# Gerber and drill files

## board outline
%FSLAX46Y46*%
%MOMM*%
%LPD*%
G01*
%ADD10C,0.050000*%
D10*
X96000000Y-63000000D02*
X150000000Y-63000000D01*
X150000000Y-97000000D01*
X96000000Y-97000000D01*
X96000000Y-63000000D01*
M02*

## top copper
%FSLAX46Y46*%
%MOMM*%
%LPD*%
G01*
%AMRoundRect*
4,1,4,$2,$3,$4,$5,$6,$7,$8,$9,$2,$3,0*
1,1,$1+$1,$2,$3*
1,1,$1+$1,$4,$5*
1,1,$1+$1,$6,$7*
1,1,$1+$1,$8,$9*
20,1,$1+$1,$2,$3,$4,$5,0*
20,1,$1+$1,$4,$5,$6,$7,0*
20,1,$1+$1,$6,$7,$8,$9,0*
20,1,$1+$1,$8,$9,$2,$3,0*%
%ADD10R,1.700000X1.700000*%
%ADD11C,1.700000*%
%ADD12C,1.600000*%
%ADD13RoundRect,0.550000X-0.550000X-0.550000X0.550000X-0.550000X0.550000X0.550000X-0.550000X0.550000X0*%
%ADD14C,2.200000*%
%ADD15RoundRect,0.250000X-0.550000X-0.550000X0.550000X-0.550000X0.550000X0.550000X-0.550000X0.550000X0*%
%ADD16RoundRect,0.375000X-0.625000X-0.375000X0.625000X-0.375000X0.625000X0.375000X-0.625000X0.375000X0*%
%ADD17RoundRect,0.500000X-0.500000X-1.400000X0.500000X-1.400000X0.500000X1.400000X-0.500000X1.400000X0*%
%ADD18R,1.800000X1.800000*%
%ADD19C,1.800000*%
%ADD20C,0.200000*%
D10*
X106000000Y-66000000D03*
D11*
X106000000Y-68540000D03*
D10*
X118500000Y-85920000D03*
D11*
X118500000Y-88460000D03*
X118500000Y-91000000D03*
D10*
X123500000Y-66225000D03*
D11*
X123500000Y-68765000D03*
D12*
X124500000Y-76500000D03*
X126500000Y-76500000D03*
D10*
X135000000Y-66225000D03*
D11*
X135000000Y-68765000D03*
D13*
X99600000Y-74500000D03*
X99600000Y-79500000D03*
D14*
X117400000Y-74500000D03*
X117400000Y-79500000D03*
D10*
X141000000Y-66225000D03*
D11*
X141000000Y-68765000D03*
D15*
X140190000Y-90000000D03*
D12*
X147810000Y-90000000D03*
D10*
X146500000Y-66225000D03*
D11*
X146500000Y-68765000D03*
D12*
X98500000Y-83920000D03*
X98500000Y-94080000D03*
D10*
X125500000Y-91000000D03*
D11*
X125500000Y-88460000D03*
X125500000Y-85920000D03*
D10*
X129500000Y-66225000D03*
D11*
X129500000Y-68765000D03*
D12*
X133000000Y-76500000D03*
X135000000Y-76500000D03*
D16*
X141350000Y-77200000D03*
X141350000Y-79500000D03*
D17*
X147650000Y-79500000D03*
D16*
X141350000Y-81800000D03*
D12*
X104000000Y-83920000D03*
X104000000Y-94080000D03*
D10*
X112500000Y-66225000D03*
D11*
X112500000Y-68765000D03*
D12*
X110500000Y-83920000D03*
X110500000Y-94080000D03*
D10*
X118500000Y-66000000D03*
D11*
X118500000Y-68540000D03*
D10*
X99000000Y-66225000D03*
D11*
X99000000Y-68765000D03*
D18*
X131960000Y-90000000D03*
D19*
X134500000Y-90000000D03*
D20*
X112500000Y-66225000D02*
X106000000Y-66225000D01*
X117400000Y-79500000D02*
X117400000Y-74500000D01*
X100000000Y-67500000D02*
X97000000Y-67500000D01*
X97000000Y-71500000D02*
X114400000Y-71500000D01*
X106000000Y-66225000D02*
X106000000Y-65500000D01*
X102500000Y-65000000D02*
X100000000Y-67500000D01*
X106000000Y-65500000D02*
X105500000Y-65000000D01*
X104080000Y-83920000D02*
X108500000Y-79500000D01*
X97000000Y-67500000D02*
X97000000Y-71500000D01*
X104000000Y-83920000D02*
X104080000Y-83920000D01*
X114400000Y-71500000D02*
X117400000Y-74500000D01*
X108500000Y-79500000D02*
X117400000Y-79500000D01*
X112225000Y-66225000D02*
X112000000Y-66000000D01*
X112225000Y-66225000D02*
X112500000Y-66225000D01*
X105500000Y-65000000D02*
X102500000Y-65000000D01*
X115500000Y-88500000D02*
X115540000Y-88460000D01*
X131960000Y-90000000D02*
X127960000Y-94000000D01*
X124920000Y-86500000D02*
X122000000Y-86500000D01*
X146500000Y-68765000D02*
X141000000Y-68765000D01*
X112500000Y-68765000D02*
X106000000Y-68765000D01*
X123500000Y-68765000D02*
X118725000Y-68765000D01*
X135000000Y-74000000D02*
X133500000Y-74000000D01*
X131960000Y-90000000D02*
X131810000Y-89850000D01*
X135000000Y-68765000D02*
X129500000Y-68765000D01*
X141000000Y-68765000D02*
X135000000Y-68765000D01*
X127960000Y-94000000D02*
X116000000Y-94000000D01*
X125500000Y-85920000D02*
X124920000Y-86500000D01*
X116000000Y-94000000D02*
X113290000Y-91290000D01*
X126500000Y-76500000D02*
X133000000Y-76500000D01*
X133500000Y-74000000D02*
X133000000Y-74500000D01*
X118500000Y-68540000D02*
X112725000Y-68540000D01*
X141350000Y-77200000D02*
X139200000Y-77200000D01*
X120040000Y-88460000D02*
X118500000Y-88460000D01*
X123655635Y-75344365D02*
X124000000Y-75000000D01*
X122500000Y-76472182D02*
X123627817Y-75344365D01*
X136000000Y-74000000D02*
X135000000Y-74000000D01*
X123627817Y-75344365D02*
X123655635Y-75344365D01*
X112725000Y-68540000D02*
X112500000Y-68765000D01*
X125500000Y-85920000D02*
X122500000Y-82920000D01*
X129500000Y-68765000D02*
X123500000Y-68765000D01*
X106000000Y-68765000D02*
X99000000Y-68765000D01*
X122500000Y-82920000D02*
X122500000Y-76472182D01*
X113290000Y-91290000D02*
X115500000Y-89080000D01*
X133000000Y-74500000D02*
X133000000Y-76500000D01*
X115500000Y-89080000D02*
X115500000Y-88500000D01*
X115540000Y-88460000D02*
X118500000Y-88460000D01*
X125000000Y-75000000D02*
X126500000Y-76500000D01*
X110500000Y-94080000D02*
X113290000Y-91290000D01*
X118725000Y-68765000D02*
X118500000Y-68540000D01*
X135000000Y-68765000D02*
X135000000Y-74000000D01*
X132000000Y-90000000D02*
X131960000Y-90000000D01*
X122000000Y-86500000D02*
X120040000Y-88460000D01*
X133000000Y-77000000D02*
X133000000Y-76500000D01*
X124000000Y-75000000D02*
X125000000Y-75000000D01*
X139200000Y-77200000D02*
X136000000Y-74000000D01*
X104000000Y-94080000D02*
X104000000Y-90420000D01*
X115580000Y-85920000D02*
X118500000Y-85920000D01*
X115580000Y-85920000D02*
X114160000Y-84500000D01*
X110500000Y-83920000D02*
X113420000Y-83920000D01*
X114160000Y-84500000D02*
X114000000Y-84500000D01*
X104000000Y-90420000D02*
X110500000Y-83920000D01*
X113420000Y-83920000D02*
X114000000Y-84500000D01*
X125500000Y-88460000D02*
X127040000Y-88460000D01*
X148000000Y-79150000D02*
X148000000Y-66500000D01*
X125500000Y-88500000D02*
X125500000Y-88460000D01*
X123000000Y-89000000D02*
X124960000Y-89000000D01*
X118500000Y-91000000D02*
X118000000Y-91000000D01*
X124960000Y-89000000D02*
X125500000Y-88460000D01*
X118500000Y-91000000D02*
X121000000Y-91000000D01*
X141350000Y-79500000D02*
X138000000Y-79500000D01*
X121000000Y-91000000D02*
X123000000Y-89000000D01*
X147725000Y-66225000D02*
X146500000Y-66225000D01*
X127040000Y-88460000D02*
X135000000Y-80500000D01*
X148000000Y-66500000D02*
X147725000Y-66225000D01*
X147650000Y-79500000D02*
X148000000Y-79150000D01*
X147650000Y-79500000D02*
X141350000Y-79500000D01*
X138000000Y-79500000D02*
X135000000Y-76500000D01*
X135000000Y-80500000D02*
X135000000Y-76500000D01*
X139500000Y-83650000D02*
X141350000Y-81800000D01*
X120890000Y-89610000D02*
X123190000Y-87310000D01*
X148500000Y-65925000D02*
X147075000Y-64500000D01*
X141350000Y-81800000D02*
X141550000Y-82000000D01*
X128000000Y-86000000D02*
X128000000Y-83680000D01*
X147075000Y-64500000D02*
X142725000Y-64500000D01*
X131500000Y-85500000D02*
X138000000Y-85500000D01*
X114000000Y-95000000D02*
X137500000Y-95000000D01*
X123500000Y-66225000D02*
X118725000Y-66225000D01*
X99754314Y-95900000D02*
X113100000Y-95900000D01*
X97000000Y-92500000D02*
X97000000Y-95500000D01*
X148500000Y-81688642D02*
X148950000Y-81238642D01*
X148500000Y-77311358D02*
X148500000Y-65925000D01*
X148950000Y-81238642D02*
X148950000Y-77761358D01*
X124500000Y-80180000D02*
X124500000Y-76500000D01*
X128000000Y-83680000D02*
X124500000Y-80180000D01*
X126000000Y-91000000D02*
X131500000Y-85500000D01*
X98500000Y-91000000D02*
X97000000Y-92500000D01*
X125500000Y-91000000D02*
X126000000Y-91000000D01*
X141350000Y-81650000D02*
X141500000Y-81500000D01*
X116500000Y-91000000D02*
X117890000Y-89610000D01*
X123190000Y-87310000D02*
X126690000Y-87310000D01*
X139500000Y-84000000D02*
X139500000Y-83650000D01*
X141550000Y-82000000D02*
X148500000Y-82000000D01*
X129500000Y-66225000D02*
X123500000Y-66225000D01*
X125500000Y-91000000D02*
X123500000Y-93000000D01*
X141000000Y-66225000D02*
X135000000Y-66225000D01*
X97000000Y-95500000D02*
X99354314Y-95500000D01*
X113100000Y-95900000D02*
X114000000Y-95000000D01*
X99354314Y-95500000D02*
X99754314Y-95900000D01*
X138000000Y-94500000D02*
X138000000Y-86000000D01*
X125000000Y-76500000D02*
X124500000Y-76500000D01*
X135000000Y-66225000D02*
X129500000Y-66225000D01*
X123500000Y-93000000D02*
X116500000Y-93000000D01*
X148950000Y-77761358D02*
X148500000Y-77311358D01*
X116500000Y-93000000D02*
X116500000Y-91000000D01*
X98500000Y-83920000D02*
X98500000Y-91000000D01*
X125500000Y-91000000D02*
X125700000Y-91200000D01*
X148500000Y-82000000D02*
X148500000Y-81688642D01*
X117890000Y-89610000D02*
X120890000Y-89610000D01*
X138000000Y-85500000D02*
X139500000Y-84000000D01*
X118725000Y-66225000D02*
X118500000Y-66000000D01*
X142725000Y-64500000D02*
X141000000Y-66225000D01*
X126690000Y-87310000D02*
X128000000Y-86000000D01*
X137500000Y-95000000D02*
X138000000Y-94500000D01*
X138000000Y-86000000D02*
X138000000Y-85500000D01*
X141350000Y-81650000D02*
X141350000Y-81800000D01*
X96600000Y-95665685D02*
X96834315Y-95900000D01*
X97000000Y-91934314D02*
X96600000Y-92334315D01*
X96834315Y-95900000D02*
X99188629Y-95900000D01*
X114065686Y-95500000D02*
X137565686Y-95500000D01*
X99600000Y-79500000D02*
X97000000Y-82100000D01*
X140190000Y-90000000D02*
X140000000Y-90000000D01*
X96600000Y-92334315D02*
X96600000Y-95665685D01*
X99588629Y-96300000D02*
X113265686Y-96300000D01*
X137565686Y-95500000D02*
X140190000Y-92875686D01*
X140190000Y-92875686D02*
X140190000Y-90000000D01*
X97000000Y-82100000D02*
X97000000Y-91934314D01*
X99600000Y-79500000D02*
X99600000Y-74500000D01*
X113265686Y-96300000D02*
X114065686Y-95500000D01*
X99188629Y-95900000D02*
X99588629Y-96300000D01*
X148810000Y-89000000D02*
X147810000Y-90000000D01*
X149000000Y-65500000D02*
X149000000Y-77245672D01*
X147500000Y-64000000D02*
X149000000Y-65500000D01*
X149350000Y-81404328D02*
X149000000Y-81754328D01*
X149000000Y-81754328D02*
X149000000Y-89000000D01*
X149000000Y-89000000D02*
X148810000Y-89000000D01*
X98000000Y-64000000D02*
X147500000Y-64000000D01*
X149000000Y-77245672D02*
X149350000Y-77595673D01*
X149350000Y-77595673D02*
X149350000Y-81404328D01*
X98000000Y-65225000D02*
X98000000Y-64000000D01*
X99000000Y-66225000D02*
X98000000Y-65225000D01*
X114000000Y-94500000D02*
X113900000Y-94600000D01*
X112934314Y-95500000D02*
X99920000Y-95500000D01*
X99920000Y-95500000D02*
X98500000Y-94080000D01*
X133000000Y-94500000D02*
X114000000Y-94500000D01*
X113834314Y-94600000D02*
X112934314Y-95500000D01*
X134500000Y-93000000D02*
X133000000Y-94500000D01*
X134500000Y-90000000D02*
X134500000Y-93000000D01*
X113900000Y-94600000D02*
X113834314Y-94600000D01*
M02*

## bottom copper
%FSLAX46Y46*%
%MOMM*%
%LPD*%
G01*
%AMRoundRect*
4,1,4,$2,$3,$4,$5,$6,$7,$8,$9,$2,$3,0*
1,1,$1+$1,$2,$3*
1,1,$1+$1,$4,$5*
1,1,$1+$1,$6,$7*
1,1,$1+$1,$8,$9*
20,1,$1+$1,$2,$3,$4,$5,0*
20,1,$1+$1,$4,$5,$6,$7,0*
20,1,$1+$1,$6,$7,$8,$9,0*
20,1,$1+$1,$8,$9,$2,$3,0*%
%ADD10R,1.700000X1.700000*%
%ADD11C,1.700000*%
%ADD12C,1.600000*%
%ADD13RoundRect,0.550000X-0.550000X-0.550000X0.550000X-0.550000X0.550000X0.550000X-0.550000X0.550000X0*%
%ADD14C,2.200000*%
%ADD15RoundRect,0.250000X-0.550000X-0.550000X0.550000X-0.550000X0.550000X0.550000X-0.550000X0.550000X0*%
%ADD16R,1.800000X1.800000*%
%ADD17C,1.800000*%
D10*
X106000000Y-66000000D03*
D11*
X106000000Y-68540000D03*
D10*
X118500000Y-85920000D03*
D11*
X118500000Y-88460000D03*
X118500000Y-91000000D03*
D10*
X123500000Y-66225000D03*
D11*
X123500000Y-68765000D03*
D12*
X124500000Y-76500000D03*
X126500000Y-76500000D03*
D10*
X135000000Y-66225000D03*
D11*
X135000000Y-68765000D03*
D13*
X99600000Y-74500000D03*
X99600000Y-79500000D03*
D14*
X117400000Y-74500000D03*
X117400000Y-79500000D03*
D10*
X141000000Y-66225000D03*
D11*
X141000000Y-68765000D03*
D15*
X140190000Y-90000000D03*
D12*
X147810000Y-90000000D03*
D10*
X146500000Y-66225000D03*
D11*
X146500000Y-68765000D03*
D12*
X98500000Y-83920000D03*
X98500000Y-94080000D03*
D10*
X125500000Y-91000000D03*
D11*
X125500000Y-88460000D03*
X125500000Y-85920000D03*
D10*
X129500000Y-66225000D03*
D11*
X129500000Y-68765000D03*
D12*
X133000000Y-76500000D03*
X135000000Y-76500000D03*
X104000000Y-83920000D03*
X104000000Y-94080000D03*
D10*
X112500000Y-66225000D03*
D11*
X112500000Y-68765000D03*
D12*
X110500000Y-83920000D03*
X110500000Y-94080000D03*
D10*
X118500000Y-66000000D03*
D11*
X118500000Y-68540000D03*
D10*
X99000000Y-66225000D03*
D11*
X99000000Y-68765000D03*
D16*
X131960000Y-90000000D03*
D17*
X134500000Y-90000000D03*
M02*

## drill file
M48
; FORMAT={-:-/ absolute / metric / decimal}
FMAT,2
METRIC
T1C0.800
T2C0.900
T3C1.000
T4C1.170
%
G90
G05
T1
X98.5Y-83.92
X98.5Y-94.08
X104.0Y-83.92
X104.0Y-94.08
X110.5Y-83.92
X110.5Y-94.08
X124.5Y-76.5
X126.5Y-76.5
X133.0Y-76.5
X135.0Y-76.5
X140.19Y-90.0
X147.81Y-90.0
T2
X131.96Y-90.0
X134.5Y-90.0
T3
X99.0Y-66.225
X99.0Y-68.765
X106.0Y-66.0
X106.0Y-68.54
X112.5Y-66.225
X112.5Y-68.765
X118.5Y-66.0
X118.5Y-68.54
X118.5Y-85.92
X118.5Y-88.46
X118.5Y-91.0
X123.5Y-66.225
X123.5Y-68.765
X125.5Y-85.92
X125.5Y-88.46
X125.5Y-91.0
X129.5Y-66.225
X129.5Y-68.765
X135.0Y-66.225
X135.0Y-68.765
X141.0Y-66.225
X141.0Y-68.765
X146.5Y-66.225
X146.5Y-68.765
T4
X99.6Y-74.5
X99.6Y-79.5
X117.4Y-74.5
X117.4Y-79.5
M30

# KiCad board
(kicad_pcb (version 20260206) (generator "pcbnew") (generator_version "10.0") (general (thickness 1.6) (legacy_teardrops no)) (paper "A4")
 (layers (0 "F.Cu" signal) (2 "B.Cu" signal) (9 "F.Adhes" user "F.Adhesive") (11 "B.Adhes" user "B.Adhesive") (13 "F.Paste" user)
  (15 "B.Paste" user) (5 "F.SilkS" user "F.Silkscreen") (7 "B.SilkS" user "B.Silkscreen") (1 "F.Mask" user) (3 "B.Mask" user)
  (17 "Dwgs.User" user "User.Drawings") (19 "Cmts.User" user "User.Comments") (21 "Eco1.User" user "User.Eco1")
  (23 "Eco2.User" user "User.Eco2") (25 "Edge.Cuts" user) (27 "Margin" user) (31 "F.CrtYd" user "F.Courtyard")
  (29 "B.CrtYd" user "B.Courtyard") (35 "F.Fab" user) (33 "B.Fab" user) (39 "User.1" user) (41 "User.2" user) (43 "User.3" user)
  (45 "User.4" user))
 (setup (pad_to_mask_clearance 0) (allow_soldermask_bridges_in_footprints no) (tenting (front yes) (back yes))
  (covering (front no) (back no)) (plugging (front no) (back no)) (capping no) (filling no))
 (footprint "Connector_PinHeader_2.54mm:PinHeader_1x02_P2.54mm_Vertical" (layer "F.Cu") (at 106 66)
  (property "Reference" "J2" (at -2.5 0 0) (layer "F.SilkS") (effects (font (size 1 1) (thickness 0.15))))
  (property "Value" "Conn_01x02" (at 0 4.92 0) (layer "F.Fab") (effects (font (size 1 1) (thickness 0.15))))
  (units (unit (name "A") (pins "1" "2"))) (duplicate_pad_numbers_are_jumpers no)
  (pad "1" thru_hole rect (at 0 0) (size 1.7 1.7) (drill 1) (layers "*.Cu" "*.Mask") (remove_unused_layers no) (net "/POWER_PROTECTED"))
  (pad "2" thru_hole circle (at 0 2.54) (size 1.7 1.7) (drill 1) (layers "*.Cu" "*.Mask") (remove_unused_layers no) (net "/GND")))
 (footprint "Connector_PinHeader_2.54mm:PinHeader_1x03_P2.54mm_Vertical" (layer "F.Cu") (at 118.5 85.92)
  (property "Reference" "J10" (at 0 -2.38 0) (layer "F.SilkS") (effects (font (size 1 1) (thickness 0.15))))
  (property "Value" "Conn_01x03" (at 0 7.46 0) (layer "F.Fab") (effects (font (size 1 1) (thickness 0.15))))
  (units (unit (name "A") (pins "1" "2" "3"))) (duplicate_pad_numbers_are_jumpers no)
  (pad "1" thru_hole rect (at 0 0) (size 1.7 1.7) (drill 1) (layers "*.Cu" "*.Mask") (remove_unused_layers no) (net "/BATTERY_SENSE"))
  (pad "2" thru_hole circle (at 0 2.54) (size 1.7 1.7) (drill 1) (layers "*.Cu" "*.Mask") (remove_unused_layers no) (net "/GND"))
  (pad "3" thru_hole circle (at 0 5.08) (size 1.7 1.7) (drill 1) (layers "*.Cu" "*.Mask") (remove_unused_layers no) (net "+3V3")))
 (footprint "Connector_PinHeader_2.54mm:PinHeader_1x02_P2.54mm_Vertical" (layer "F.Cu") (at 123.5 66.225)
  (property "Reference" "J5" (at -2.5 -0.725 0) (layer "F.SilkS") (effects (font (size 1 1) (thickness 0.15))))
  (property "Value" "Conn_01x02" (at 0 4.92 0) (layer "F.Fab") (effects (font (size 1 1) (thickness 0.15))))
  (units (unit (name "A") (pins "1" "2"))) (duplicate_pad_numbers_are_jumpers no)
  (pad "1" thru_hole rect (at 0 0) (size 1.7 1.7) (drill 1) (layers "*.Cu" "*.Mask") (remove_unused_layers no) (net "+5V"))
  (pad "2" thru_hole circle (at 0 2.54) (size 1.7 1.7) (drill 1) (layers "*.Cu" "*.Mask") (remove_unused_layers no) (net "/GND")))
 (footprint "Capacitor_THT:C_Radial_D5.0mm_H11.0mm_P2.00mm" (layer "F.Cu") (at 124.5 76.5)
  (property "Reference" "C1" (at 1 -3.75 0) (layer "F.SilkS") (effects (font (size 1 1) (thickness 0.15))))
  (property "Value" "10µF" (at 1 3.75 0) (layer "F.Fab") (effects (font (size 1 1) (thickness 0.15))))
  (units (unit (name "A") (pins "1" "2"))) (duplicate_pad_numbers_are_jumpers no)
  (pad "1" thru_hole circle (at 0 0) (size 1.6 1.6) (drill 0.8) (layers "*.Cu" "*.Mask") (remove_unused_layers no) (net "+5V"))
  (pad "2" thru_hole circle (at 2 0) (size 1.6 1.6) (drill 0.8) (layers "*.Cu" "*.Mask") (remove_unused_layers no) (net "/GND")))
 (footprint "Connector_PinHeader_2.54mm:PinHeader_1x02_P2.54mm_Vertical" (layer "F.Cu") (at 135 66.225)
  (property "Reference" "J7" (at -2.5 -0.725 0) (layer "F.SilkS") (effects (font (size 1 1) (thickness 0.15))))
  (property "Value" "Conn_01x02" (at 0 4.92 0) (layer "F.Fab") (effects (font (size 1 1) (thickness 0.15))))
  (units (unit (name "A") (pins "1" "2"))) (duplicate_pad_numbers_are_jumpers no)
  (pad "1" thru_hole rect (at 0 0) (size 1.7 1.7) (drill 1) (layers "*.Cu" "*.Mask") (remove_unused_layers no) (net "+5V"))
  (pad "2" thru_hole circle (at 0 2.54) (size 1.7 1.7) (drill 1) (layers "*.Cu" "*.Mask") (remove_unused_layers no) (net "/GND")))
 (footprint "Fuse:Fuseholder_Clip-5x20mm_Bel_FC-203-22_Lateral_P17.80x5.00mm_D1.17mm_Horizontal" (layer "F.Cu") (at 99.6 74.5)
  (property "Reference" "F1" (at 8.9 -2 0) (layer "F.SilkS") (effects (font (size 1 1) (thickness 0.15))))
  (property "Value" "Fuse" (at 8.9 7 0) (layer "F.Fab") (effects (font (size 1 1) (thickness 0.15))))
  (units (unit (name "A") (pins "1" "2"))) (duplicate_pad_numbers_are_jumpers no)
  (pad "1" thru_hole roundrect (at 0 0) (size 2.2 2.2) (drill 1.17) (layers "*.Cu" "*.Mask") (remove_unused_layers no)
   (roundrect_rratio 0.25) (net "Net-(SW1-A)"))
  (pad "1" thru_hole roundrect (at 0 5) (size 2.2 2.2) (drill 1.17) (layers "*.Cu" "*.Mask") (remove_unused_layers no)
   (roundrect_rratio 0.25) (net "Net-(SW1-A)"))
  (pad "2" thru_hole circle (at 17.8 0) (size 2.2 2.2) (drill 1.17) (layers "*.Cu" "*.Mask") (remove_unused_layers no)
   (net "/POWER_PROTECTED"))
  (pad "2" thru_hole circle (at 17.8 5) (size 2.2 2.2) (drill 1.17) (layers "*.Cu" "*.Mask") (remove_unused_layers no)
   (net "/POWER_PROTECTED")))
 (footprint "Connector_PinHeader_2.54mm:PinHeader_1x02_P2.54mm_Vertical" (layer "F.Cu") (at 141 66.225)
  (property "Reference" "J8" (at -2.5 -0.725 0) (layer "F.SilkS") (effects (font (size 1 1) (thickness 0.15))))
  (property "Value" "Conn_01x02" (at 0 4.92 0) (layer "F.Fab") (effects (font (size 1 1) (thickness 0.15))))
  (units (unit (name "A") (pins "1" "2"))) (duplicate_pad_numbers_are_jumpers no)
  (pad "1" thru_hole rect (at 0 0) (size 1.7 1.7) (drill 1) (layers "*.Cu" "*.Mask") (remove_unused_layers no) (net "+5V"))
  (pad "2" thru_hole circle (at 0 2.54) (size 1.7 1.7) (drill 1) (layers "*.Cu" "*.Mask") (remove_unused_layers no) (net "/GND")))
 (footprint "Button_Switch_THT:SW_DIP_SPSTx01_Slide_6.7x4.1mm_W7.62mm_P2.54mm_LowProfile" (layer "F.Cu") (at 140.19 90)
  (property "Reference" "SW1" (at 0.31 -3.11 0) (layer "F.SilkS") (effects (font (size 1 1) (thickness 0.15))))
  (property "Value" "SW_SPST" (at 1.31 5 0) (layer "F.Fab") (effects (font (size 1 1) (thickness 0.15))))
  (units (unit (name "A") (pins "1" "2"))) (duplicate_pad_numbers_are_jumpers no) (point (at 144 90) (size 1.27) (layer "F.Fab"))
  (pad "1" thru_hole roundrect (at 0 0) (size 1.6 1.6) (drill 0.8) (layers "*.Cu" "*.Mask") (remove_unused_layers no)
   (roundrect_rratio 0.15625) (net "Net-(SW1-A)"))
  (pad "2" thru_hole circle (at 7.62 0) (size 1.6 1.6) (drill 0.8) (layers "*.Cu" "*.Mask") (remove_unused_layers no) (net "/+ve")))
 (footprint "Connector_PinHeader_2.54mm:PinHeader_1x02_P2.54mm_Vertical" (layer "F.Cu") (at 146.5 66.225)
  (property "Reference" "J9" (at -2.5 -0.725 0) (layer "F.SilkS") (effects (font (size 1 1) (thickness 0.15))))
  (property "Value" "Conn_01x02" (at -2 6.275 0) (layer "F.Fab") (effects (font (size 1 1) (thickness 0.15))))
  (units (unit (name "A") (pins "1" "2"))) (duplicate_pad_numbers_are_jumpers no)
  (pad "1" thru_hole rect (at 0 0) (size 1.7 1.7) (drill 1) (layers "*.Cu" "*.Mask") (remove_unused_layers no) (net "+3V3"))
  (pad "2" thru_hole circle (at 0 2.54) (size 1.7 1.7) (drill 1) (layers "*.Cu" "*.Mask") (remove_unused_layers no) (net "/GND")))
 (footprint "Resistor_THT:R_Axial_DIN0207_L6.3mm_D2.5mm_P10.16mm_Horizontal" (layer "F.Cu") (at 98.5 83.92 -90)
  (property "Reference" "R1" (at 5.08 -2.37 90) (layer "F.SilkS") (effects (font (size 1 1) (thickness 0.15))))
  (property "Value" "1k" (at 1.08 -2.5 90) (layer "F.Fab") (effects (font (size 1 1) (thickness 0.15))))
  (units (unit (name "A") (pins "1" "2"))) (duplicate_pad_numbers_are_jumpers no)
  (pad "1" thru_hole circle (at 0 0 270) (size 1.6 1.6) (drill 0.8) (layers "*.Cu" "*.Mask") (remove_unused_layers no) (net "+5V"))
  (pad "2" thru_hole circle (at 10.16 0 270) (size 1.6 1.6) (drill 0.8) (layers "*.Cu" "*.Mask") (remove_unused_layers no)
   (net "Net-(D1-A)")))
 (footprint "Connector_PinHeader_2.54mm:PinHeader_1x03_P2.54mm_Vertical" (layer "F.Cu") (at 125.5 91 180)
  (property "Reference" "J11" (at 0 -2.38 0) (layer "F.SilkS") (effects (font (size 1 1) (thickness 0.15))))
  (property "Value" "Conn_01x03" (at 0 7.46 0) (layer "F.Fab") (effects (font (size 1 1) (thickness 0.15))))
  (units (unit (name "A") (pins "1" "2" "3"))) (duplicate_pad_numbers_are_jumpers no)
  (pad "1" thru_hole rect (at 0 0 180) (size 1.7 1.7) (drill 1) (layers "*.Cu" "*.Mask") (remove_unused_layers no) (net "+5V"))
  (pad "2" thru_hole circle (at 0 2.54 180) (size 1.7 1.7) (drill 1) (layers "*.Cu" "*.Mask") (remove_unused_layers no) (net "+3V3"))
  (pad "3" thru_hole circle (at 0 5.08 180) (size 1.7 1.7) (drill 1) (layers "*.Cu" "*.Mask") (remove_unused_layers no) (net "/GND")))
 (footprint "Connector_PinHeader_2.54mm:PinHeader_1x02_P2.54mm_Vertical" (layer "F.Cu") (at 129.5 66.225)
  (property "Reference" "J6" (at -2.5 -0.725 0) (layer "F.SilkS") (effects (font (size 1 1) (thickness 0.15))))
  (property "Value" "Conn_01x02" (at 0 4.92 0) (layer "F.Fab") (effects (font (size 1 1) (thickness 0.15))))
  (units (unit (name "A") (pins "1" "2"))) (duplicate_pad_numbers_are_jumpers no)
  (pad "1" thru_hole rect (at 0 0) (size 1.7 1.7) (drill 1) (layers "*.Cu" "*.Mask") (remove_unused_layers no) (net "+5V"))
  (pad "2" thru_hole circle (at 0 2.54) (size 1.7 1.7) (drill 1) (layers "*.Cu" "*.Mask") (remove_unused_layers no) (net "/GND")))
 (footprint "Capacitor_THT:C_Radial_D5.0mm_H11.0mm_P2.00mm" (layer "F.Cu") (at 133 76.5)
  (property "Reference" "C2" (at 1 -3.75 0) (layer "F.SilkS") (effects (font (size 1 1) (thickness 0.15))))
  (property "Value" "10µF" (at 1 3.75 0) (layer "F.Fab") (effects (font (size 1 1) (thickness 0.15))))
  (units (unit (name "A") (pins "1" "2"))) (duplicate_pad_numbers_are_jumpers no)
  (pad "1" thru_hole circle (at 0 0) (size 1.6 1.6) (drill 0.8) (layers "*.Cu" "*.Mask") (remove_unused_layers no) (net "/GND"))
  (pad "2" thru_hole circle (at 2 0) (size 1.6 1.6) (drill 0.8) (layers "*.Cu" "*.Mask") (remove_unused_layers no) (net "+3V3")))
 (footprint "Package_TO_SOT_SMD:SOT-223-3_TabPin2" (layer "F.Cu") (at 144.5 79.5)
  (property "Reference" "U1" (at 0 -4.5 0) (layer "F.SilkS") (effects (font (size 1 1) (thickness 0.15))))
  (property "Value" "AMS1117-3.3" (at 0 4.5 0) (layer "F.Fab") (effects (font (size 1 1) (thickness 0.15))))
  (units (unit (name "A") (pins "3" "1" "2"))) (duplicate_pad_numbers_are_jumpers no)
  (pad "1" smd roundrect (at -3.15 -2.3) (size 2 1.5) (layers "F.Cu" "F.Mask" "F.Paste") (roundrect_rratio 0.25) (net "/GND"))
  (pad "2" smd roundrect (at -3.15 0) (size 2 1.5) (layers "F.Cu" "F.Mask" "F.Paste") (roundrect_rratio 0.25) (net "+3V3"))
  (pad "2" smd roundrect (at 3.15 0) (size 2 3.8) (layers "F.Cu" "F.Mask" "F.Paste") (roundrect_rratio 0.25) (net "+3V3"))
  (pad "3" smd roundrect (at -3.15 2.3) (size 2 1.5) (layers "F.Cu" "F.Mask" "F.Paste") (roundrect_rratio 0.25) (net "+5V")))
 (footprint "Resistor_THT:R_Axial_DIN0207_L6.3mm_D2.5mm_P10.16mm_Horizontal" (layer "F.Cu") (at 104 83.92 -90)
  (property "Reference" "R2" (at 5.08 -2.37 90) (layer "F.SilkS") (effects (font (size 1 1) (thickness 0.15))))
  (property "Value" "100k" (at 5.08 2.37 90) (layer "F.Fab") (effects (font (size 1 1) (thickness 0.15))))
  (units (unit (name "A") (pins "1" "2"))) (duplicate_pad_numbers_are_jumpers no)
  (pad "1" thru_hole circle (at 0 0 270) (size 1.6 1.6) (drill 0.8) (layers "*.Cu" "*.Mask") (remove_unused_layers no)
   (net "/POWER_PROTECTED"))
  (pad "2" thru_hole circle (at 10.16 0 270) (size 1.6 1.6) (drill 0.8) (layers "*.Cu" "*.Mask") (remove_unused_layers no)
   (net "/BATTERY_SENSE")))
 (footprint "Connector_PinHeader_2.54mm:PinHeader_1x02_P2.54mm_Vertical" (layer "F.Cu") (at 112.5 66.225)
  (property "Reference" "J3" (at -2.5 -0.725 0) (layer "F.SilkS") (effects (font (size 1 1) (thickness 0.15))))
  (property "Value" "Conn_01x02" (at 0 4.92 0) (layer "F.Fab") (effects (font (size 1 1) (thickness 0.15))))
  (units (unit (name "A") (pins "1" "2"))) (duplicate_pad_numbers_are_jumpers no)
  (pad "1" thru_hole rect (at 0 0) (size 1.7 1.7) (drill 1) (layers "*.Cu" "*.Mask") (remove_unused_layers no) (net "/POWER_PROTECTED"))
  (pad "2" thru_hole circle (at 0 2.54) (size 1.7 1.7) (drill 1) (layers "*.Cu" "*.Mask") (remove_unused_layers no) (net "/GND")))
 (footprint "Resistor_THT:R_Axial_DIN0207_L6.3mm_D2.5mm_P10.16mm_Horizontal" (layer "F.Cu") (at 110.5 83.92 -90)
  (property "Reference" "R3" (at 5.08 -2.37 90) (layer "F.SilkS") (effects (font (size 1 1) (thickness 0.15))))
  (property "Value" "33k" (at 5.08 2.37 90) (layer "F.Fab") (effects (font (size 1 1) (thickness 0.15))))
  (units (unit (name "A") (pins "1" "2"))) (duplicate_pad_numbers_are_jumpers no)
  (pad "1" thru_hole circle (at 0 0 270) (size 1.6 1.6) (drill 0.8) (layers "*.Cu" "*.Mask") (remove_unused_layers no)
   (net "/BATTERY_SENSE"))
  (pad "2" thru_hole circle (at 10.16 0 270) (size 1.6 1.6) (drill 0.8) (layers "*.Cu" "*.Mask") (remove_unused_layers no) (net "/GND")))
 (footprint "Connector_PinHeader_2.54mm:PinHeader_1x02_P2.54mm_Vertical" (layer "F.Cu") (at 118.5 66)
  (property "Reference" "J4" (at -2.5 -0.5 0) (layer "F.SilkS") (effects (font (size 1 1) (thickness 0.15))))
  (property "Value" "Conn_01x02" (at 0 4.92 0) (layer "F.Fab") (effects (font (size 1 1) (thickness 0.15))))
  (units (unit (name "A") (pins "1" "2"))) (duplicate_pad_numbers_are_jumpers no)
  (pad "1" thru_hole rect (at 0 0) (size 1.7 1.7) (drill 1) (layers "*.Cu" "*.Mask") (remove_unused_layers no) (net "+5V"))
  (pad "2" thru_hole circle (at 0 2.54) (size 1.7 1.7) (drill 1) (layers "*.Cu" "*.Mask") (remove_unused_layers no) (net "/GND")))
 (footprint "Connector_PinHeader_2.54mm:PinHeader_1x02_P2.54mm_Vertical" (layer "F.Cu") (at 99 66.225)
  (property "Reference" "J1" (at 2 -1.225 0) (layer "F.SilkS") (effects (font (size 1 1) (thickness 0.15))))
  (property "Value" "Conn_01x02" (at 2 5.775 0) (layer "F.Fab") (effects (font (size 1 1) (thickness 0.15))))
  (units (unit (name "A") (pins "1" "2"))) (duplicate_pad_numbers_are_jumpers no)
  (pad "1" thru_hole rect (at 0 0) (size 1.7 1.7) (drill 1) (layers "*.Cu" "*.Mask") (remove_unused_layers no) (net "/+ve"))
  (pad "2" thru_hole circle (at 0 2.54) (size 1.7 1.7) (drill 1) (layers "*.Cu" "*.Mask") (remove_unused_layers no) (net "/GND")))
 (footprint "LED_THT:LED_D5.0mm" (layer "F.Cu") (at 131.96 90)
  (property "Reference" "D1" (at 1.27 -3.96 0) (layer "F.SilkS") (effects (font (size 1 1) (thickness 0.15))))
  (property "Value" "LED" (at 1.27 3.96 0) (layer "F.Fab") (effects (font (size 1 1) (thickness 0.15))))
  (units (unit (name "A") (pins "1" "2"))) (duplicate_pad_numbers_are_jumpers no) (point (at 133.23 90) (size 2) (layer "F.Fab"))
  (pad "1" thru_hole rect (at 0 0) (size 1.8 1.8) (drill 0.9) (layers "*.Cu" "*.Mask") (remove_unused_layers no) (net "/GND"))
  (pad "2" thru_hole circle (at 2.54 0) (size 1.8 1.8) (drill 0.9) (layers "*.Cu" "*.Mask") (remove_unused_layers no) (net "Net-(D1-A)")))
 (gr_rect (start 96 63) (end 150 97) (stroke (width 0.05) (type solid)) (fill no) (layer "Edge.Cuts"))
 (segment (start 112.5 66.225) (end 106 66.225) (width 0.2) (layer "F.Cu") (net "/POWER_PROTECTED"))
 (segment (start 117.4 79.5) (end 117.4 74.5) (width 0.2) (layer "F.Cu") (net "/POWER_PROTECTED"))
 (segment (start 100 67.5) (end 97 67.5) (width 0.2) (layer "F.Cu") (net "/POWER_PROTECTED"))
 (segment (start 97 71.5) (end 114.4 71.5) (width 0.2) (layer "F.Cu") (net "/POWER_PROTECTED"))
 (segment (start 106 66.225) (end 106 65.5) (width 0.2) (layer "F.Cu") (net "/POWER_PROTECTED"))
 (segment (start 102.5 65) (end 100 67.5) (width 0.2) (layer "F.Cu") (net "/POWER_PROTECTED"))
 (segment (start 106 65.5) (end 105.5 65) (width 0.2) (layer "F.Cu") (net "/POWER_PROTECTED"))
 (segment (start 104.08 83.92) (end 108.5 79.5) (width 0.2) (layer "F.Cu") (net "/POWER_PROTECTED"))
 (segment (start 97 67.5) (end 97 71.5) (width 0.2) (layer "F.Cu") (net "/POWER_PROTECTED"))
 (segment (start 104 83.92) (end 104.08 83.92) (width 0.2) (layer "F.Cu") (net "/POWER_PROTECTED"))
 (segment (start 114.4 71.5) (end 117.4 74.5) (width 0.2) (layer "F.Cu") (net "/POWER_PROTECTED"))
 (segment (start 108.5 79.5) (end 117.4 79.5) (width 0.2) (layer "F.Cu") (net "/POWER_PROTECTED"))
 (segment (start 112.225 66.225) (end 112 66) (width 0.2) (layer "F.Cu") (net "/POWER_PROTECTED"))
 (segment (start 112.225 66.225) (end 112.5 66.225) (width 0.2) (layer "F.Cu") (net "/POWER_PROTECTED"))
 (segment (start 105.5 65) (end 102.5 65) (width 0.2) (layer "F.Cu") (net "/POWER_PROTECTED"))
 (segment (start 115.5 88.5) (end 115.54 88.46) (width 0.2) (layer "F.Cu") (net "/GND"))
 (segment (start 131.96 90) (end 127.96 94) (width 0.2) (layer "F.Cu") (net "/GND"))
 (segment (start 124.92 86.5) (end 122 86.5) (width 0.2) (layer "F.Cu") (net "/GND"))
 (segment (start 146.5 68.765) (end 141 68.765) (width 0.2) (layer "F.Cu") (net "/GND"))
 (segment (start 112.5 68.765) (end 106 68.765) (width 0.2) (layer "F.Cu") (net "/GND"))
 (segment (start 123.5 68.765) (end 118.725 68.765) (width 0.2) (layer "F.Cu") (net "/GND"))
 (segment (start 135 74) (end 133.5 74) (width 0.2) (layer "F.Cu") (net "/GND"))
 (segment (start 131.96 90) (end 131.81 89.85) (width 0.2) (layer "F.Cu") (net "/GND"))
 (segment (start 135 68.765) (end 129.5 68.765) (width 0.2) (layer "F.Cu") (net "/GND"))
 (segment (start 141 68.765) (end 135 68.765) (width 0.2) (layer "F.Cu") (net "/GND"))
 (segment (start 127.96 94) (end 116 94) (width 0.2) (layer "F.Cu") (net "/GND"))
 (segment (start 125.5 85.92) (end 124.92 86.5) (width 0.2) (layer "F.Cu") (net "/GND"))
 (segment (start 116 94) (end 113.29 91.29) (width 0.2) (layer "F.Cu") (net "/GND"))
 (segment (start 126.5 76.5) (end 133 76.5) (width 0.2) (layer "F.Cu") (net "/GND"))
 (segment (start 133.5 74) (end 133 74.5) (width 0.2) (layer "F.Cu") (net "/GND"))
 (segment (start 118.5 68.54) (end 112.725 68.54) (width 0.2) (layer "F.Cu") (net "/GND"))
 (segment (start 141.35 77.2) (end 139.2 77.2) (width 0.2) (layer "F.Cu") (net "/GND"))
 (segment (start 120.04 88.46) (end 118.5 88.46) (width 0.2) (layer "F.Cu") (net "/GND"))
 (segment (start 123.655635 75.344365) (end 124 75) (width 0.2) (layer "F.Cu") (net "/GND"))
 (segment (start 122.5 76.472182) (end 123.627817 75.344365) (width 0.2) (layer "F.Cu") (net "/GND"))
 (segment (start 136 74) (end 135 74) (width 0.2) (layer "F.Cu") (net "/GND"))
 (segment (start 123.627817 75.344365) (end 123.655635 75.344365) (width 0.2) (layer "F.Cu") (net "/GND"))
 (segment (start 112.725 68.54) (end 112.5 68.765) (width 0.2) (layer "F.Cu") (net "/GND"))
 (segment (start 125.5 85.92) (end 122.5 82.92) (width 0.2) (layer "F.Cu") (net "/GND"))
 (segment (start 129.5 68.765) (end 123.5 68.765) (width 0.2) (layer "F.Cu") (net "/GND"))
 (segment (start 106 68.765) (end 99 68.765) (width 0.2) (layer "F.Cu") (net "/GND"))
 (segment (start 122.5 82.92) (end 122.5 76.472182) (width 0.2) (layer "F.Cu") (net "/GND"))
 (segment (start 113.29 91.29) (end 115.5 89.08) (width 0.2) (layer "F.Cu") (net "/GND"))
 (segment (start 133 74.5) (end 133 76.5) (width 0.2) (layer "F.Cu") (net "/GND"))
 (segment (start 115.5 89.08) (end 115.5 88.5) (width 0.2) (layer "F.Cu") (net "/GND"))
 (segment (start 115.54 88.46) (end 118.5 88.46) (width 0.2) (layer "F.Cu") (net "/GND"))
 (segment (start 125 75) (end 126.5 76.5) (width 0.2) (layer "F.Cu") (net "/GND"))
 (segment (start 110.5 94.08) (end 113.29 91.29) (width 0.2) (layer "F.Cu") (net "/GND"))
 (segment (start 118.725 68.765) (end 118.5 68.54) (width 0.2) (layer "F.Cu") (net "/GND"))
 (segment (start 135 68.765) (end 135 74) (width 0.2) (layer "F.Cu") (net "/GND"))
 (segment (start 132 90) (end 131.96 90) (width 0.2) (layer "F.Cu") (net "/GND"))
 (segment (start 122 86.5) (end 120.04 88.46) (width 0.2) (layer "F.Cu") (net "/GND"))
 (segment (start 133 77) (end 133 76.5) (width 0.2) (layer "F.Cu") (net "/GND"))
 (segment (start 124 75) (end 125 75) (width 0.2) (layer "F.Cu") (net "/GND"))
 (segment (start 139.2 77.2) (end 136 74) (width 0.2) (layer "F.Cu") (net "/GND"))
 (segment (start 104 94.08) (end 104 90.42) (width 0.2) (layer "F.Cu") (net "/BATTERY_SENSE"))
 (segment (start 115.58 85.92) (end 118.5 85.92) (width 0.2) (layer "F.Cu") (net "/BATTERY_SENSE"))
 (segment (start 115.58 85.92) (end 114.16 84.5) (width 0.2) (layer "F.Cu") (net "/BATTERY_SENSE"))
 (segment (start 110.5 83.92) (end 113.42 83.92) (width 0.2) (layer "F.Cu") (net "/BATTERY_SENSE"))
 (segment (start 114.16 84.5) (end 114 84.5) (width 0.2) (layer "F.Cu") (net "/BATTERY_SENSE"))
 (segment (start 104 90.42) (end 110.5 83.92) (width 0.2) (layer "F.Cu") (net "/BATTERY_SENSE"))
 (segment (start 113.42 83.92) (end 114 84.5) (width 0.2) (layer "F.Cu") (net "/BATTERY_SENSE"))
 (segment (start 125.5 88.46) (end 127.04 88.46) (width 0.2) (layer "F.Cu") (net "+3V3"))
 (segment (start 148 79.15) (end 148 66.5) (width 0.2) (layer "F.Cu") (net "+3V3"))
 (segment (start 125.5 88.5) (end 125.5 88.46) (width 0.2) (layer "F.Cu") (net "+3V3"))
 (segment (start 123 89) (end 124.96 89) (width 0.2) (layer "F.Cu") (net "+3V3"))
 (segment (start 118.5 91) (end 118 91) (width 0.2) (layer "F.Cu") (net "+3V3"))
 (segment (start 124.96 89) (end 125.5 88.46) (width 0.2) (layer "F.Cu") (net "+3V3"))
 (segment (start 118.5 91) (end 121 91) (width 0.2) (layer "F.Cu") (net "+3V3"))
 (segment (start 141.35 79.5) (end 138 79.5) (width 0.2) (layer "F.Cu") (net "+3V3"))
 (segment (start 121 91) (end 123 89) (width 0.2) (layer "F.Cu") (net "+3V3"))
 (segment (start 147.725 66.225) (end 146.5 66.225) (width 0.2) (layer "F.Cu") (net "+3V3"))
 (segment (start 127.04 88.46) (end 135 80.5) (width 0.2) (layer "F.Cu") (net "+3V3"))
 (segment (start 148 66.5) (end 147.725 66.225) (width 0.2) (layer "F.Cu") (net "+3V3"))
 (segment (start 147.65 79.5) (end 148 79.15) (width 0.2) (layer "F.Cu") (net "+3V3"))
 (segment (start 147.65 79.5) (end 141.35 79.5) (width 0.2) (layer "F.Cu") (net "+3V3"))
 (segment (start 138 79.5) (end 135 76.5) (width 0.2) (layer "F.Cu") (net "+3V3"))
 (segment (start 135 80.5) (end 135 76.5) (width 0.2) (layer "F.Cu") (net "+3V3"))
 (segment (start 139.5 83.65) (end 141.35 81.8) (width 0.2) (layer "F.Cu") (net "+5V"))
 (segment (start 120.89 89.61) (end 123.19 87.31) (width 0.2) (layer "F.Cu") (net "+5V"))
 (segment (start 148.5 65.925) (end 147.075 64.5) (width 0.2) (layer "F.Cu") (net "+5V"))
 (segment (start 141.35 81.8) (end 141.55 82) (width 0.2) (layer "F.Cu") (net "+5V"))
 (segment (start 128 86) (end 128 83.68) (width 0.2) (layer "F.Cu") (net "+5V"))
 (segment (start 147.075 64.5) (end 142.725 64.5) (width 0.2) (layer "F.Cu") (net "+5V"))
 (segment (start 131.5 85.5) (end 138 85.5) (width 0.2) (layer "F.Cu") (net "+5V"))
 (segment (start 114 95) (end 137.5 95) (width 0.2) (layer "F.Cu") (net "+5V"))
 (segment (start 123.5 66.225) (end 118.725 66.225) (width 0.2) (layer "F.Cu") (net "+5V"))
 (segment (start 99.754314 95.9) (end 113.1 95.9) (width 0.2) (layer "F.Cu") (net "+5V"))
 (segment (start 97 92.5) (end 97 95.5) (width 0.2) (layer "F.Cu") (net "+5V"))
 (segment (start 148.5 81.688642) (end 148.95 81.238642) (width 0.2) (layer "F.Cu") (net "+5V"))
 (segment (start 148.5 77.311358) (end 148.5 65.925) (width 0.2) (layer "F.Cu") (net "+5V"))
 (segment (start 148.95 81.238642) (end 148.95 77.761358) (width 0.2) (layer "F.Cu") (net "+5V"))
 (segment (start 124.5 80.18) (end 124.5 76.5) (width 0.2) (layer "F.Cu") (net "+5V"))
 (segment (start 128 83.68) (end 124.5 80.18) (width 0.2) (layer "F.Cu") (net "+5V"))
 (segment (start 126 91) (end 131.5 85.5) (width 0.2) (layer "F.Cu") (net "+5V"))
 (segment (start 98.5 91) (end 97 92.5) (width 0.2) (layer "F.Cu") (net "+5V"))
 (segment (start 125.5 91) (end 126 91) (width 0.2) (layer "F.Cu") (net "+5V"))
 (segment (start 141.35 81.65) (end 141.5 81.5) (width 0.2) (layer "F.Cu") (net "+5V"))
 (segment (start 116.5 91) (end 117.89 89.61) (width 0.2) (layer "F.Cu") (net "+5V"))
 (segment (start 123.19 87.31) (end 126.69 87.31) (width 0.2) (layer "F.Cu") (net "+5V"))
 (segment (start 139.5 84) (end 139.5 83.65) (width 0.2) (layer "F.Cu") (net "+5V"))
 (segment (start 141.55 82) (end 148.5 82) (width 0.2) (layer "F.Cu") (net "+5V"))
 (segment (start 129.5 66.225) (end 123.5 66.225) (width 0.2) (layer "F.Cu") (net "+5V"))
 (segment (start 125.5 91) (end 123.5 93) (width 0.2) (layer "F.Cu") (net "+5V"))
 (segment (start 141 66.225) (end 135 66.225) (width 0.2) (layer "F.Cu") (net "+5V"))
 (segment (start 97 95.5) (end 99.354314 95.5) (width 0.2) (layer "F.Cu") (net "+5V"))
 (segment (start 113.1 95.9) (end 114 95) (width 0.2) (layer "F.Cu") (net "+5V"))
 (segment (start 99.354314 95.5) (end 99.754314 95.9) (width 0.2) (layer "F.Cu") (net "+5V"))
 (segment (start 138 94.5) (end 138 86) (width 0.2) (layer "F.Cu") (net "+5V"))
 (segment (start 125 76.5) (end 124.5 76.5) (width 0.2) (layer "F.Cu") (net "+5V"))
 (segment (start 135 66.225) (end 129.5 66.225) (width 0.2) (layer "F.Cu") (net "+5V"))
 (segment (start 123.5 93) (end 116.5 93) (width 0.2) (layer "F.Cu") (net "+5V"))
 (segment (start 148.95 77.761358) (end 148.5 77.311358) (width 0.2) (layer "F.Cu") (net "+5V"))
 (segment (start 116.5 93) (end 116.5 91) (width 0.2) (layer "F.Cu") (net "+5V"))
 (segment (start 98.5 83.92) (end 98.5 91) (width 0.2) (layer "F.Cu") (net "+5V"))
 (segment (start 125.5 91) (end 125.7 91.2) (width 0.2) (layer "F.Cu") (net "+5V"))
 (segment (start 148.5 82) (end 148.5 81.688642) (width 0.2) (layer "F.Cu") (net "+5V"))
 (segment (start 117.89 89.61) (end 120.89 89.61) (width 0.2) (layer "F.Cu") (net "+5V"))
 (segment (start 138 85.5) (end 139.5 84) (width 0.2) (layer "F.Cu") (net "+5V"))
 (segment (start 118.725 66.225) (end 118.5 66) (width 0.2) (layer "F.Cu") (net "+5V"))
 (segment (start 142.725 64.5) (end 141 66.225) (width 0.2) (layer "F.Cu") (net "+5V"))
 (segment (start 126.69 87.31) (end 128 86) (width 0.2) (layer "F.Cu") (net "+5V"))
 (segment (start 137.5 95) (end 138 94.5) (width 0.2) (layer "F.Cu") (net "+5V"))
 (segment (start 138 86) (end 138 85.5) (width 0.2) (layer "F.Cu") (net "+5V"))
 (segment (start 141.35 81.65) (end 141.35 81.8) (width 0.2) (layer "F.Cu") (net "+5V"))
 (segment (start 96.6 95.665685) (end 96.834315 95.9) (width 0.2) (layer "F.Cu") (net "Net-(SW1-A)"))
 (segment (start 97 91.934314) (end 96.6 92.334315) (width 0.2) (layer "F.Cu") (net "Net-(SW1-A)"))
 (segment (start 96.834315 95.9) (end 99.188629 95.9) (width 0.2) (layer "F.Cu") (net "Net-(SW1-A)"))
 (segment (start 114.065686 95.5) (end 137.565686 95.5) (width 0.2) (layer "F.Cu") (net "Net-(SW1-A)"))
 (segment (start 99.6 79.5) (end 97 82.1) (width 0.2) (layer "F.Cu") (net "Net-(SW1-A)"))
 (segment (start 140.19 90) (end 140 90) (width 0.2) (layer "F.Cu") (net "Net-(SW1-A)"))
 (segment (start 96.6 92.334315) (end 96.6 95.665685) (width 0.2) (layer "F.Cu") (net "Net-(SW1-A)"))
 (segment (start 99.588629 96.3) (end 113.265686 96.3) (width 0.2) (layer "F.Cu") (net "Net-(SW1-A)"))
 (segment (start 137.565686 95.5) (end 140.19 92.875686) (width 0.2) (layer "F.Cu") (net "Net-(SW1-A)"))
 (segment (start 140.19 92.875686) (end 140.19 90) (width 0.2) (layer "F.Cu") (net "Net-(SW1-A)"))
 (segment (start 97 82.1) (end 97 91.934314) (width 0.2) (layer "F.Cu") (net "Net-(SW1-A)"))
 (segment (start 99.6 79.5) (end 99.6 74.5) (width 0.2) (layer "F.Cu") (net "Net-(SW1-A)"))
 (segment (start 113.265686 96.3) (end 114.065686 95.5) (width 0.2) (layer "F.Cu") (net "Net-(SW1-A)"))
 (segment (start 99.188629 95.9) (end 99.588629 96.3) (width 0.2) (layer "F.Cu") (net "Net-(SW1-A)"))
 (segment (start 148.81 89) (end 147.81 90) (width 0.2) (layer "F.Cu") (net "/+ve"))
 (segment (start 149 65.5) (end 149 77.245672) (width 0.2) (layer "F.Cu") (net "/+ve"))
 (segment (start 147.5 64) (end 149 65.5) (width 0.2) (layer "F.Cu") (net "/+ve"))
 (segment (start 149.35 81.404328) (end 149 81.754328) (width 0.2) (layer "F.Cu") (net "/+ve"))
 (segment (start 149 81.754328) (end 149 89) (width 0.2) (layer "F.Cu") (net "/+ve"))
 (segment (start 149 89) (end 148.81 89) (width 0.2) (layer "F.Cu") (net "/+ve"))
 (segment (start 98 64) (end 147.5 64) (width 0.2) (layer "F.Cu") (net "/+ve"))
 (segment (start 149 77.245672) (end 149.35 77.595673) (width 0.2) (layer "F.Cu") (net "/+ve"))
 (segment (start 149.35 77.595673) (end 149.35 81.404328) (width 0.2) (layer "F.Cu") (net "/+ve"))
 (segment (start 98 65.225) (end 98 64) (width 0.2) (layer "F.Cu") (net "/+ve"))
 (segment (start 99 66.225) (end 98 65.225) (width 0.2) (layer "F.Cu") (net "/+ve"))
 (segment (start 114 94.5) (end 113.9 94.6) (width 0.2) (layer "F.Cu") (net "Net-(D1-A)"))
 (segment (start 112.934314 95.5) (end 99.92 95.5) (width 0.2) (layer "F.Cu") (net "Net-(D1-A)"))
 (segment (start 99.92 95.5) (end 98.5 94.08) (width 0.2) (layer "F.Cu") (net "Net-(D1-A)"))
 (segment (start 133 94.5) (end 114 94.5) (width 0.2) (layer "F.Cu") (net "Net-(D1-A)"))
 (segment (start 113.834314 94.6) (end 112.934314 95.5) (width 0.2) (layer "F.Cu") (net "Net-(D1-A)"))
 (segment (start 134.5 93) (end 133 94.5) (width 0.2) (layer "F.Cu") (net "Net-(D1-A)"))
 (segment (start 134.5 90) (end 134.5 93) (width 0.2) (layer "F.Cu") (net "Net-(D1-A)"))
 (segment (start 113.9 94.6) (end 113.834314 94.6) (width 0.2) (layer "F.Cu") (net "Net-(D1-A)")))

